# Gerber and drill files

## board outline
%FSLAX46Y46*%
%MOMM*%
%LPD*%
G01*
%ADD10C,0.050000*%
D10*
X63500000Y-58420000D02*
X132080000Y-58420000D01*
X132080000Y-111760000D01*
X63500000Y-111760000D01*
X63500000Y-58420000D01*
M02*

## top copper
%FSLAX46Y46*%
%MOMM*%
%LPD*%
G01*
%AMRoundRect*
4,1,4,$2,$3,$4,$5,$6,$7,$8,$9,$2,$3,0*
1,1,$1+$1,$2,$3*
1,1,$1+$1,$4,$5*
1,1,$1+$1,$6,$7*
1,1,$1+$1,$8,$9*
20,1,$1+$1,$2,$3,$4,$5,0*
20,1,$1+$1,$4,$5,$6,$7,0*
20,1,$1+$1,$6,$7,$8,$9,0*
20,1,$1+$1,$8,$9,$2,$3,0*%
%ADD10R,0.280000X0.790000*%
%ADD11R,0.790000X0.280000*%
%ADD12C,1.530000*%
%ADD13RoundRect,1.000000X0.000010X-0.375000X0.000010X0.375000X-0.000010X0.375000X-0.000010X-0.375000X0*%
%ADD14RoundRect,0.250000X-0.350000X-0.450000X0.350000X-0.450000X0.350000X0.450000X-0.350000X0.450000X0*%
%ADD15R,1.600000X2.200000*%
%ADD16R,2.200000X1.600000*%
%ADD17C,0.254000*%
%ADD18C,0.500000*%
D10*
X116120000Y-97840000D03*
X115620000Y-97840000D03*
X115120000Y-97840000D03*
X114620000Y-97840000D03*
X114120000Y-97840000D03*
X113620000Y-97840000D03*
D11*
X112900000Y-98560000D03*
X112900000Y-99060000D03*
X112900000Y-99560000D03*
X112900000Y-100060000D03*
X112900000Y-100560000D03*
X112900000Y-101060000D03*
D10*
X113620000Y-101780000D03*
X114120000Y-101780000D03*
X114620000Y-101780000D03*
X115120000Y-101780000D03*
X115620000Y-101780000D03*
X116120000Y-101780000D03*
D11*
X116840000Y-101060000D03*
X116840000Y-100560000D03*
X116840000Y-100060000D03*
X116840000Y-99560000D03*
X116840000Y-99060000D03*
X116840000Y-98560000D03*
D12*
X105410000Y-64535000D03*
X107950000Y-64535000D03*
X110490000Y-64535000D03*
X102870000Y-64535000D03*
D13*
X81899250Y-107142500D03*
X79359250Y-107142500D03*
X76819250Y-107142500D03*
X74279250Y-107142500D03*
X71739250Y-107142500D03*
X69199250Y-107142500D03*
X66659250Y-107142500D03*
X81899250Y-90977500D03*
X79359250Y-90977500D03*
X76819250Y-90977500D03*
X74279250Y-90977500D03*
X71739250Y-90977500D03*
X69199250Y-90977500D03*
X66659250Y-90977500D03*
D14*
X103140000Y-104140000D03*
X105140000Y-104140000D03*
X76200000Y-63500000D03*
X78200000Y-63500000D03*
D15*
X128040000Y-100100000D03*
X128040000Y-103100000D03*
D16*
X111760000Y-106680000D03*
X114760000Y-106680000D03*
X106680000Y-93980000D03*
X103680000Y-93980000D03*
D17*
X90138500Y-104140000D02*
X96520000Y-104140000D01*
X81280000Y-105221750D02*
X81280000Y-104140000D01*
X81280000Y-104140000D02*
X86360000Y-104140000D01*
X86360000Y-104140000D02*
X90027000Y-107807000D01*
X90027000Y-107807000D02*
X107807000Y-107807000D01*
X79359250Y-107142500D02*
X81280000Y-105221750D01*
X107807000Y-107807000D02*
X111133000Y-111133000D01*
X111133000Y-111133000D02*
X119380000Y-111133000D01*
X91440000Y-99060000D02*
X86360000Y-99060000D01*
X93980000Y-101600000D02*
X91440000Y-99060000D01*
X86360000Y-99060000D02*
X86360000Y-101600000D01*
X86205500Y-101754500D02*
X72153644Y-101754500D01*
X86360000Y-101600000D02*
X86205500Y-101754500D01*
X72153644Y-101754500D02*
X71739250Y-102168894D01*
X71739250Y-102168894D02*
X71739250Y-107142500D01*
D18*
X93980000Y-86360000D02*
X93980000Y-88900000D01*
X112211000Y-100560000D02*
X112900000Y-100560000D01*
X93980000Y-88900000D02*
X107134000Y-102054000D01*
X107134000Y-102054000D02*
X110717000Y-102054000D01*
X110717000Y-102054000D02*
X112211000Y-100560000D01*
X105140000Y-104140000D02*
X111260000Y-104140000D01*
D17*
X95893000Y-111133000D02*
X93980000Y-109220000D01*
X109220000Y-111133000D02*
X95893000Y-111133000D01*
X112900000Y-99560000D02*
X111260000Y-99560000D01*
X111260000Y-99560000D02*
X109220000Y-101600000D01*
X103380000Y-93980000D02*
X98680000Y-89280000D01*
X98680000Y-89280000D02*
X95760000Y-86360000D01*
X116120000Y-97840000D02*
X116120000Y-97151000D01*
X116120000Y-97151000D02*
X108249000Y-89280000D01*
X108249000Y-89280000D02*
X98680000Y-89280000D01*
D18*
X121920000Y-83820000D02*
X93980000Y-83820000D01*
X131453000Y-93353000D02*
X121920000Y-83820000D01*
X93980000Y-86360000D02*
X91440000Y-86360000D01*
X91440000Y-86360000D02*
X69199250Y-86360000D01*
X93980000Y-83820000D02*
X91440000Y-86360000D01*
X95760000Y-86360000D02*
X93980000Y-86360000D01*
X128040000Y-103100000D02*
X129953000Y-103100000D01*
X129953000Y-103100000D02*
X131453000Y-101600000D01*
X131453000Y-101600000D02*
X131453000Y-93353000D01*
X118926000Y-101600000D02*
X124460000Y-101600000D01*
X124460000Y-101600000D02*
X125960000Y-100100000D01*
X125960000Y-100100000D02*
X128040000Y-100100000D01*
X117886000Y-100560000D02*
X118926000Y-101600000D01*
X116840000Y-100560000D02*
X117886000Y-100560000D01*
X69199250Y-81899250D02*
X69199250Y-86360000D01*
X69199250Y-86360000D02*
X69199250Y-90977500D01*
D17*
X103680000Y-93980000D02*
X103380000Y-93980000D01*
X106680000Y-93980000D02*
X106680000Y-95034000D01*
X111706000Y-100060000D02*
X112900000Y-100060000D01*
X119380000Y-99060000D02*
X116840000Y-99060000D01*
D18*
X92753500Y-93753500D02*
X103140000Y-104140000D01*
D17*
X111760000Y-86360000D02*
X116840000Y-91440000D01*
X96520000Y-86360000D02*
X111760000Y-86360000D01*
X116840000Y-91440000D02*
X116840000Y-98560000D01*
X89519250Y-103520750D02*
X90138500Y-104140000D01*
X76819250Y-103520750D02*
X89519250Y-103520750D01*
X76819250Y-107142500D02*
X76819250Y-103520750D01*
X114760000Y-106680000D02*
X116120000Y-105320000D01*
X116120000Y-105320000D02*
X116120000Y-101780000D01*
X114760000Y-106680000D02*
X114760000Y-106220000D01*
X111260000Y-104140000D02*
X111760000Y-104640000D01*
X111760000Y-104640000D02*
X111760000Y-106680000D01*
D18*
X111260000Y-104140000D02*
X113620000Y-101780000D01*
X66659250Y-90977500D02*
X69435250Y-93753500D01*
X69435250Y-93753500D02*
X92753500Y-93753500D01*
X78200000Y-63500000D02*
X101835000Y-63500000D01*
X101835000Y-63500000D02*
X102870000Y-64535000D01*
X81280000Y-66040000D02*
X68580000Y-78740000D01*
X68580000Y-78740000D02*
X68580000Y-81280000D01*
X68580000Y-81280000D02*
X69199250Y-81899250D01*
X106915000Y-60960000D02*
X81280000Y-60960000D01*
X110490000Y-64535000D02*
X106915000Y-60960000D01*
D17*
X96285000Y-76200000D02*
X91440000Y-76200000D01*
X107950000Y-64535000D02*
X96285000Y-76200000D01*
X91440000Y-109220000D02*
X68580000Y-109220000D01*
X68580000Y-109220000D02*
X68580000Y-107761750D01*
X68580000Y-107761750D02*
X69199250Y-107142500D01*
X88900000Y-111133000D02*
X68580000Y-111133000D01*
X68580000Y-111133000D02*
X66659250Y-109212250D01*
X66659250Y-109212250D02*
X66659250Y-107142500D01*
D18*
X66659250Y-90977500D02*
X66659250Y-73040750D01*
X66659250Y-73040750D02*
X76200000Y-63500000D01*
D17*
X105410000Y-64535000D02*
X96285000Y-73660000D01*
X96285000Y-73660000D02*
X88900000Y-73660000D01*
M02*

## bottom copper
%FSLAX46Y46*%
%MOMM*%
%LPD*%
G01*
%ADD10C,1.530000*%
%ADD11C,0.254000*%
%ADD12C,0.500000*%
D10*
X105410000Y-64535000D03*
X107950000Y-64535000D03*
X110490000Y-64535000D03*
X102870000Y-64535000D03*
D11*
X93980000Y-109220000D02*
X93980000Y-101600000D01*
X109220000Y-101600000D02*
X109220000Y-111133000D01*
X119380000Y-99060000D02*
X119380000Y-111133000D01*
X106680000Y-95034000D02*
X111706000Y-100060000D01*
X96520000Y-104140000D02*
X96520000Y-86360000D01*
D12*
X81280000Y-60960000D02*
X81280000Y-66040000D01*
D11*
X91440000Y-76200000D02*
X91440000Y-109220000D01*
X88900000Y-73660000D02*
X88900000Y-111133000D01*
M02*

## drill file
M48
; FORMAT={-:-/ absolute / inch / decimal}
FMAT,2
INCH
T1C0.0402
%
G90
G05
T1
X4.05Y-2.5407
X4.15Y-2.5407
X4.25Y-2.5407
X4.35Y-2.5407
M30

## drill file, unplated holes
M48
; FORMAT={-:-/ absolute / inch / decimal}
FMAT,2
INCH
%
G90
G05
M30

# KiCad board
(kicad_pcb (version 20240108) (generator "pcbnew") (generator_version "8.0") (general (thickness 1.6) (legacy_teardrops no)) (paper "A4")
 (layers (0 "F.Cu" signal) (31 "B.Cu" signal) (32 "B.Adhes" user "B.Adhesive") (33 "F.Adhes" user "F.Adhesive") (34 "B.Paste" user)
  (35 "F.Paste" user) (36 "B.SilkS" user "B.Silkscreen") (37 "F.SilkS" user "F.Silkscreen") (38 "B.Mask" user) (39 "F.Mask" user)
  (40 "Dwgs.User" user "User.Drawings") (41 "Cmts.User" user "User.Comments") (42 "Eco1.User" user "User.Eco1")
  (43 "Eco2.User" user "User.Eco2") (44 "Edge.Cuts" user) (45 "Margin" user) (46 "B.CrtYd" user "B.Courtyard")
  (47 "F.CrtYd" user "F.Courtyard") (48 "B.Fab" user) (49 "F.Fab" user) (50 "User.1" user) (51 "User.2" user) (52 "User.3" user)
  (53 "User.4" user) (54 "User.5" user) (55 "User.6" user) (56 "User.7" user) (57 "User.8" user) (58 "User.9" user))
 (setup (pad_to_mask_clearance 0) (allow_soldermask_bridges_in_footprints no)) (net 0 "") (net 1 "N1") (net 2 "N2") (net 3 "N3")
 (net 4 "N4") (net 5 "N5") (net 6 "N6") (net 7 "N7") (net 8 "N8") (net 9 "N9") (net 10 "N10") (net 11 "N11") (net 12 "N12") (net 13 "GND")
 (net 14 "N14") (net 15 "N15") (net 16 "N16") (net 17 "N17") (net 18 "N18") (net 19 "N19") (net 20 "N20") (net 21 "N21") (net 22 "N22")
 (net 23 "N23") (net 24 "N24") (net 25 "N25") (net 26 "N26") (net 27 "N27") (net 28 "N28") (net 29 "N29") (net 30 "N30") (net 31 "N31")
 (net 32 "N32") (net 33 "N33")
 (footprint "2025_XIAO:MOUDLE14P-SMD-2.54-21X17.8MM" (layer "F.Cu") (at 84.77925 107.9775 90)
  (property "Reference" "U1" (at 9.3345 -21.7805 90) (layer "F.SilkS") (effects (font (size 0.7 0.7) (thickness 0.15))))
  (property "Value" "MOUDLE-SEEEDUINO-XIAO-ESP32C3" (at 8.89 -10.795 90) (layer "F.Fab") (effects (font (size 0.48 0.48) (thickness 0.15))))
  (pad "1" smd roundrect (at 0.835 -18.12 90) (size 2.75 2) (layers "F.Cu" "F.Paste" "F.Mask") (roundrect_rratio 0.5) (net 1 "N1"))
  (pad "2" smd roundrect (at 0.835 -15.58 90) (size 2.75 2) (layers "F.Cu" "F.Paste" "F.Mask") (roundrect_rratio 0.5) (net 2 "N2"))
  (pad "3" smd roundrect (at 0.835 -13.04 90) (size 2.75 2) (layers "F.Cu" "F.Paste" "F.Mask") (roundrect_rratio 0.5) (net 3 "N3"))
  (pad "4" smd roundrect (at 0.835 -10.5 90) (size 2.75 2) (layers "F.Cu" "F.Paste" "F.Mask") (roundrect_rratio 0.5) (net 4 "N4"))
  (pad "5" smd roundrect (at 0.835 -7.96 90) (size 2.75 2) (layers "F.Cu" "F.Paste" "F.Mask") (roundrect_rratio 0.5) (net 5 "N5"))
  (pad "6" smd roundrect (at 0.835 -5.42 90) (size 2.75 2) (layers "F.Cu" "F.Paste" "F.Mask") (roundrect_rratio 0.5) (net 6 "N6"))
  (pad "7" smd roundrect (at 0.835 -2.88 90) (size 2.75 2) (layers "F.Cu" "F.Paste" "F.Mask") (roundrect_rratio 0.5) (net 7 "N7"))
  (pad "8" smd roundrect (at 17 -2.88 90) (size 2.75 2) (layers "F.Cu" "F.Paste" "F.Mask") (roundrect_rratio 0.5) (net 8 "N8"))
  (pad "9" smd roundrect (at 17 -5.42 90) (size 2.75 2) (layers "F.Cu" "F.Paste" "F.Mask") (roundrect_rratio 0.5) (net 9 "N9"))
  (pad "10" smd roundrect (at 17 -7.96 90) (size 2.75 2) (layers "F.Cu" "F.Paste" "F.Mask") (roundrect_rratio 0.5) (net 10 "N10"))
  (pad "11" smd roundrect (at 17 -10.5 90) (size 2.75 2) (layers "F.Cu" "F.Paste" "F.Mask") (roundrect_rratio 0.5) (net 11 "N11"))
  (pad "12" smd roundrect (at 17 -13.04 90) (size 2.75 2) (layers "F.Cu" "F.Paste" "F.Mask") (roundrect_rratio 0.5) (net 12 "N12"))
  (pad "13" smd roundrect (at 17 -15.58 90) (size 2.75 2) (layers "F.Cu" "F.Paste" "F.Mask") (roundrect_rratio 0.5) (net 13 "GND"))
  (pad "14" smd roundrect (at 17 -18.12 90) (size 2.75 2) (layers "F.Cu" "F.Paste" "F.Mask") (roundrect_rratio 0.5) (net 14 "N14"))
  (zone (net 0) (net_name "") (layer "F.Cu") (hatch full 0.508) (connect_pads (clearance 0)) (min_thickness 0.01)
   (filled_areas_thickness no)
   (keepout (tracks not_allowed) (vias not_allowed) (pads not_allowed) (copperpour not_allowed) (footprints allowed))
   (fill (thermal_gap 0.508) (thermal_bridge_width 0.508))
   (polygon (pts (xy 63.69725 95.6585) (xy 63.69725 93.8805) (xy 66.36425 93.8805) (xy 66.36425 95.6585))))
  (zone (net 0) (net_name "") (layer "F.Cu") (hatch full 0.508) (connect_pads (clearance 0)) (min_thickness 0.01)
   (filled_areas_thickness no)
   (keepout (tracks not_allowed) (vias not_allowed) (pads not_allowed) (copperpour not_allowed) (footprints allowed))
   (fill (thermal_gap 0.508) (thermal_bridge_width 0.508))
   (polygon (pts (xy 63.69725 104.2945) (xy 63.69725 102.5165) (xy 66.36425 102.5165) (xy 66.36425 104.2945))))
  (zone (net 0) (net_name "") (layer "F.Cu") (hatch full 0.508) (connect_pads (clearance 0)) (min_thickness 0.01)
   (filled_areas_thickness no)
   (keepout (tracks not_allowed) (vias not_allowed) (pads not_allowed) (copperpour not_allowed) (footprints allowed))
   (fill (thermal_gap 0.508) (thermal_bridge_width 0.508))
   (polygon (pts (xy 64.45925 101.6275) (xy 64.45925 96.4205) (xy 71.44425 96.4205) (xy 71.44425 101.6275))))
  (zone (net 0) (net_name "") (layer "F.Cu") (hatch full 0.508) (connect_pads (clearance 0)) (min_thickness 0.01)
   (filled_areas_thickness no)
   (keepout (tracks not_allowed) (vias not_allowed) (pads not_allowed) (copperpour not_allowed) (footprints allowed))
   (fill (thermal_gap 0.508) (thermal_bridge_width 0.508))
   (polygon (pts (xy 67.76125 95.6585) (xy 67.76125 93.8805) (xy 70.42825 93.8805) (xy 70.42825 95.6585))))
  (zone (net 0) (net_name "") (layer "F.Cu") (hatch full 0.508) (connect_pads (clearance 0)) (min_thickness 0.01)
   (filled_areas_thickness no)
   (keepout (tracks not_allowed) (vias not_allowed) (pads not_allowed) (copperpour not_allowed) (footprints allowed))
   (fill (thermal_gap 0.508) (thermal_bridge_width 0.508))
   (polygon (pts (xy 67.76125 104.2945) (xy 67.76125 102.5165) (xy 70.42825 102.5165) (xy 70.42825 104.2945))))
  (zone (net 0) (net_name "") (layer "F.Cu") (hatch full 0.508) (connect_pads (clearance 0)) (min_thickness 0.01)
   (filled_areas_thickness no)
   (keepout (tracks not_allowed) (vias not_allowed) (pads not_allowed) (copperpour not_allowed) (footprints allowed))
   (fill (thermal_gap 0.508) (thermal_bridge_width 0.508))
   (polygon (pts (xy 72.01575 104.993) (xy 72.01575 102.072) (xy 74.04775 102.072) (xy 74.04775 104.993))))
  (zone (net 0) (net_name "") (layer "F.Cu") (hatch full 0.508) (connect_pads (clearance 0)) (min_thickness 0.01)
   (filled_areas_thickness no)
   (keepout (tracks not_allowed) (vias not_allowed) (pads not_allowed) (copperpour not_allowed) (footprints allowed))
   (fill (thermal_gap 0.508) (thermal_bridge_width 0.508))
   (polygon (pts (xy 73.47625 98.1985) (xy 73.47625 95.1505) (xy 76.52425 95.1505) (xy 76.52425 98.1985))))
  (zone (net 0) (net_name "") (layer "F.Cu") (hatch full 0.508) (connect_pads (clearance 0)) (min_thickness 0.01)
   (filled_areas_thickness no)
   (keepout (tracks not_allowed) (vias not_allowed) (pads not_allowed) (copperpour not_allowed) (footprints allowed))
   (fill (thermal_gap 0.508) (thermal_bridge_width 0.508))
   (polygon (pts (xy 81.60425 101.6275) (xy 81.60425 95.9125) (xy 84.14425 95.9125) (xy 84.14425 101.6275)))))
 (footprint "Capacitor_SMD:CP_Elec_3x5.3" (layer "F.Cu") (at 113.26 106.68)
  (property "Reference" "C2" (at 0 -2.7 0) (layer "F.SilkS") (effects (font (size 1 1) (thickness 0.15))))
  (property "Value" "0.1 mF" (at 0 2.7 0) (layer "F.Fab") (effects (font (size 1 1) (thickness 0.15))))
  (pad "1" smd rect (at -1.5 0) (size 2.2 1.6) (layers "F.Cu" "F.Paste" "F.Mask") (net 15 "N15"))
  (pad "2" smd rect (at 1.5 0) (size 2.2 1.6) (layers "F.Cu" "F.Paste" "F.Mask") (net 13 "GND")))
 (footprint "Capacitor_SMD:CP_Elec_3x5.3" (layer "F.Cu") (at 128.04 101.6 -90)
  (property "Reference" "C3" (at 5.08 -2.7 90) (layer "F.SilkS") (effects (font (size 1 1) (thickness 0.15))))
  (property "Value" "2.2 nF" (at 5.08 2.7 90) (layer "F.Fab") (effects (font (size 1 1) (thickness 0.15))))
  (pad "1" smd rect (at -1.5 0 270) (size 2.2 1.6) (layers "F.Cu" "F.Paste" "F.Mask") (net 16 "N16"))
  (pad "2" smd rect (at 1.5 0 270) (size 2.2 1.6) (layers "F.Cu" "F.Paste" "F.Mask") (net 13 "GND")))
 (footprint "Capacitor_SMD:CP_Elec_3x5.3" (layer "F.Cu") (at 105.18 93.98 180)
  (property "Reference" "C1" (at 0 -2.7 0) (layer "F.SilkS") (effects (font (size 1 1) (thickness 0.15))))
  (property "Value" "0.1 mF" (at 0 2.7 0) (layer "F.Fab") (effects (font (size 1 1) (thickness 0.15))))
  (pad "1" smd rect (at -1.5 0 180) (size 2.2 1.6) (layers "F.Cu" "F.Paste" "F.Mask") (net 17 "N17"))
  (pad "2" smd rect (at 1.5 0 180) (size 2.2 1.6) (layers "F.Cu" "F.Paste" "F.Mask") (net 13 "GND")))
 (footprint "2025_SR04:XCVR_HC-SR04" (layer "F.Cu") (at 106.68 64.535)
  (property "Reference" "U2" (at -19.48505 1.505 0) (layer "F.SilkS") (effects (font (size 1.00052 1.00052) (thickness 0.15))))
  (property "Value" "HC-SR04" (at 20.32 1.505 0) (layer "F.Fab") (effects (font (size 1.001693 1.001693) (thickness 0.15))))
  (pad "1" thru_hole circle (at -3.81 0) (size 1.53 1.53) (drill 1.02) (layers "*.Cu" "*.Mask") (remove_unused_layers no) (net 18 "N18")
   (solder_mask_margin 0.102))
  (pad "2" thru_hole circle (at -1.27 0) (size 1.53 1.53) (drill 1.02) (layers "*.Cu" "*.Mask") (remove_unused_layers no) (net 1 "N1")
   (solder_mask_margin 0.102))
  (pad "3" thru_hole circle (at 1.27 0) (size 1.53 1.53) (drill 1.02) (layers "*.Cu" "*.Mask") (remove_unused_layers no) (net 2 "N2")
   (solder_mask_margin 0.102))
  (pad "4" thru_hole circle (at 3.81 0) (size 1.53 1.53) (drill 1.02) (layers "*.Cu" "*.Mask") (remove_unused_layers no) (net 13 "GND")
   (solder_mask_margin 0.102)))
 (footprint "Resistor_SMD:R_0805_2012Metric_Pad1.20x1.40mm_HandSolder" (layer "F.Cu") (at 77.2 63.5)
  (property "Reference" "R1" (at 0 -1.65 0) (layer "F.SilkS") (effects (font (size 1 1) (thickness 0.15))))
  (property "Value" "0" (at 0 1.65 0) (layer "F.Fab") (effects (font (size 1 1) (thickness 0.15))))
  (pad "1" smd roundrect (at -1 0) (size 1.2 1.4) (layers "F.Cu" "F.Paste" "F.Mask") (roundrect_rratio 0.208333) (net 14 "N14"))
  (pad "2" smd roundrect (at 1 0) (size 1.2 1.4) (layers "F.Cu" "F.Paste" "F.Mask") (roundrect_rratio 0.208333) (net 18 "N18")))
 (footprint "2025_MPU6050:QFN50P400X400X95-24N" (layer "F.Cu") (at 114.87 99.81 -90)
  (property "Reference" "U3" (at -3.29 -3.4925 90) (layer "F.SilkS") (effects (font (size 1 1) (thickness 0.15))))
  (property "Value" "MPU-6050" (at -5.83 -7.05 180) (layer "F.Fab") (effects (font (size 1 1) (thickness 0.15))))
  (pad "1" smd rect (at -1.97 -1.25 270) (size 0.79 0.28) (layers "F.Cu" "F.Paste" "F.Mask") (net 13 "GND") (solder_mask_margin 0.102))
  (pad "2" smd rect (at -1.97 -0.75 270) (size 0.79 0.28) (layers "F.Cu" "F.Paste" "F.Mask") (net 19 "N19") (solder_mask_margin 0.102))
  (pad "3" smd rect (at -1.97 -0.25 270) (size 0.79 0.28) (layers "F.Cu" "F.Paste" "F.Mask") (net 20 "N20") (solder_mask_margin 0.102))
  (pad "4" smd rect (at -1.97 0.25 270) (size 0.79 0.28) (layers "F.Cu" "F.Paste" "F.Mask") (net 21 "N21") (solder_mask_margin 0.102))
  (pad "5" smd rect (at -1.97 0.75 270) (size 0.79 0.28) (layers "F.Cu" "F.Paste" "F.Mask") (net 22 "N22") (solder_mask_margin 0.102))
  (pad "6" smd rect (at -1.97 1.25 270) (size 0.79 0.28) (layers "F.Cu" "F.Paste" "F.Mask") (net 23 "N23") (solder_mask_margin 0.102))
  (pad "7" smd rect (at -1.25 1.97 270) (size 0.28 0.79) (layers "F.Cu" "F.Paste" "F.Mask") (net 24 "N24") (solder_mask_margin 0.102))
  (pad "8" smd rect (at -0.75 1.97 270) (size 0.28 0.79) (layers "F.Cu" "F.Paste" "F.Mask") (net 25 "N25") (solder_mask_margin 0.102))
  (pad "9" smd rect (at -0.25 1.97 270) (size 0.28 0.79) (layers "F.Cu" "F.Paste" "F.Mask") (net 3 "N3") (solder_mask_margin 0.102))
  (pad "10" smd rect (at 0.25 1.97 270) (size 0.28 0.79) (layers "F.Cu" "F.Paste" "F.Mask") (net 17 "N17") (solder_mask_margin 0.102))
  (pad "11" smd rect (at 0.75 1.97 270) (size 0.28 0.79) (layers "F.Cu" "F.Paste" "F.Mask") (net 13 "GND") (solder_mask_margin 0.102))
  (pad "12" smd rect (at 1.25 1.97 270) (size 0.28 0.79) (layers "F.Cu" "F.Paste" "F.Mask") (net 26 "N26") (solder_mask_margin 0.102))
  (pad "13" smd rect (at 1.97 1.25 270) (size 0.79 0.28) (layers "F.Cu" "F.Paste" "F.Mask") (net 15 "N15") (solder_mask_margin 0.102))
  (pad "14" smd rect (at 1.97 0.75 270) (size 0.79 0.28) (layers "F.Cu" "F.Paste" "F.Mask") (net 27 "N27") (solder_mask_margin 0.102))
  (pad "15" smd rect (at 1.97 0.25 270) (size 0.79 0.28) (layers "F.Cu" "F.Paste" "F.Mask") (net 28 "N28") (solder_mask_margin 0.102))
  (pad "16" smd rect (at 1.97 -0.25 270) (size 0.79 0.28) (layers "F.Cu" "F.Paste" "F.Mask") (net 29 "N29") (solder_mask_margin 0.102))
  (pad "17" smd rect (at 1.97 -0.75 270) (size 0.79 0.28) (layers "F.Cu" "F.Paste" "F.Mask") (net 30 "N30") (solder_mask_margin 0.102))
  (pad "18" smd rect (at 1.97 -1.25 270) (size 0.79 0.28) (layers "F.Cu" "F.Paste" "F.Mask") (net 13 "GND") (solder_mask_margin 0.102))
  (pad "19" smd rect (at 1.25 -1.97 270) (size 0.28 0.79) (layers "F.Cu" "F.Paste" "F.Mask") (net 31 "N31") (solder_mask_margin 0.102))
  (pad "20" smd rect (at 0.75 -1.97 270) (size 0.28 0.79) (layers "F.Cu" "F.Paste" "F.Mask") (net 16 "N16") (solder_mask_margin 0.102))
  (pad "21" smd rect (at 0.25 -1.97 270) (size 0.28 0.79) (layers "F.Cu" "F.Paste" "F.Mask") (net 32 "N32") (solder_mask_margin 0.102))
  (pad "22" smd rect (at -0.25 -1.97 270) (size 0.28 0.79) (layers "F.Cu" "F.Paste" "F.Mask") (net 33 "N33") (solder_mask_margin 0.102))
  (pad "23" smd rect (at -0.75 -1.97 270) (size 0.28 0.79) (layers "F.Cu" "F.Paste" "F.Mask") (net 6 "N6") (solder_mask_margin 0.102))
  (pad "24" smd rect (at -1.25 -1.97 270) (size 0.28 0.79) (layers "F.Cu" "F.Paste" "F.Mask") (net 5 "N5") (solder_mask_margin 0.102))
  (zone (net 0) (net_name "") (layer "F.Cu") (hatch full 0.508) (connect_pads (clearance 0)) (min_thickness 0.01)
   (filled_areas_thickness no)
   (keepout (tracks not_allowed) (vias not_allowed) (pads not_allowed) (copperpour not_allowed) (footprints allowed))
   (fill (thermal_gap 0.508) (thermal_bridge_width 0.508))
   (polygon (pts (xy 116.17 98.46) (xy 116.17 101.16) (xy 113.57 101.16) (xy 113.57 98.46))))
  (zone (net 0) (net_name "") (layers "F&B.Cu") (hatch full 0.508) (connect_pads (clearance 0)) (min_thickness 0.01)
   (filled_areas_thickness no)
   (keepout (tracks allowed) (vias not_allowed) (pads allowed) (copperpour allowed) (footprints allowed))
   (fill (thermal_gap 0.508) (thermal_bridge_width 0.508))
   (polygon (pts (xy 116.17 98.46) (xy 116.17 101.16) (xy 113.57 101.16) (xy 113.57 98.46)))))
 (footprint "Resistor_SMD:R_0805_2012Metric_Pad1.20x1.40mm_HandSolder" (layer "F.Cu") (at 104.14 104.14)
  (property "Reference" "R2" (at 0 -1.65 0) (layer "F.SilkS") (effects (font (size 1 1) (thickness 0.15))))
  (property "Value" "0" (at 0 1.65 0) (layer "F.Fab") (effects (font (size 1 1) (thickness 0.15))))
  (pad "1" smd roundrect (at -1 0) (size 1.2 1.4) (layers "F.Cu" "F.Paste" "F.Mask") (roundrect_rratio 0.208333) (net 14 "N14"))
  (pad "2" smd roundrect (at 1 0) (size 1.2 1.4) (layers "F.Cu" "F.Paste" "F.Mask") (roundrect_rratio 0.208333) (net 15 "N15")))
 (gr_rect (start 63.5 58.42) (end 132.08 111.76) (stroke (width 0.05) (type default)) (fill none) (layer "Edge.Cuts"))
 (segment (start 105.41 64.535) (end 96.285 73.66) (width 0.254) (layer "F.Cu") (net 1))
 (segment (start 88.9 111.133) (end 68.58 111.133) (width 0.254) (layer "F.Cu") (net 1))
 (segment (start 66.65925 109.21225) (end 66.65925 107.1425) (width 0.254) (layer "F.Cu") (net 1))
 (segment (start 68.58 111.133) (end 66.65925 109.21225) (width 0.254) (layer "F.Cu") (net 1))
 (segment (start 96.285 73.66) (end 88.9 73.66) (width 0.254) (layer "F.Cu") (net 1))
 (segment (start 88.9 73.66) (end 88.9 111.133) (width 0.254) (layer "B.Cu") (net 1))
 (segment (start 96.285 76.2) (end 91.44 76.2) (width 0.254) (layer "F.Cu") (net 2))
 (segment (start 91.44 109.22) (end 68.58 109.22) (width 0.254) (layer "F.Cu") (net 2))
 (segment (start 68.58 107.76175) (end 69.19925 107.1425) (width 0.254) (layer "F.Cu") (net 2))
 (segment (start 68.58 109.22) (end 68.58 107.76175) (width 0.254) (layer "F.Cu") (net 2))
 (segment (start 107.95 64.535) (end 96.285 76.2) (width 0.254) (layer "F.Cu") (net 2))
 (segment (start 91.44 76.2) (end 91.44 109.22) (width 0.254) (layer "B.Cu") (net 2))
 (segment (start 101.835 63.5) (end 102.87 64.535) (width 0.5) (layer "F.Cu") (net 18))
 (segment (start 78.2 63.5) (end 101.835 63.5) (width 0.5) (layer "F.Cu") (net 18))
 (segment (start 68.58 81.28) (end 69.19925 81.89925) (width 0.5) (layer "F.Cu") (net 13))
 (segment (start 112.211 100.56) (end 112.9 100.56) (width 0.5) (layer "F.Cu") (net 13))
 (segment (start 81.28 66.04) (end 68.58 78.74) (width 0.5) (layer "F.Cu") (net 13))
 (segment (start 106.915 60.96) (end 81.28 60.96) (width 0.5) (layer "F.Cu") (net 13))
 (segment (start 69.19925 86.36) (end 69.19925 90.9775) (width 0.5) (layer "F.Cu") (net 13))
 (segment (start 93.98 88.9) (end 107.134 102.054) (width 0.5) (layer "F.Cu") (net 13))
 (segment (start 93.98 86.36) (end 93.98 88.9) (width 0.5) (layer "F.Cu") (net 13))
 (segment (start 131.453 101.6) (end 131.453 93.353) (width 0.5) (layer "F.Cu") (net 13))
 (segment (start 116.12 97.151) (end 108.249 89.28) (width 0.254) (layer "F.Cu") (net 13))
 (segment (start 116.12 105.32) (end 116.12 101.78) (width 0.254) (layer "F.Cu") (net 13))
 (segment (start 116.12 97.84) (end 116.12 97.151) (width 0.254) (layer "F.Cu") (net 13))
 (segment (start 108.249 89.28) (end 98.68 89.28) (width 0.254) (layer "F.Cu") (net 13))
 (segment (start 121.92 83.82) (end 93.98 83.82) (width 0.5) (layer "F.Cu") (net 13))
 (segment (start 93.98 86.36) (end 91.44 86.36) (width 0.5) (layer "F.Cu") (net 13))
 (segment (start 98.68 89.28) (end 95.76 86.36) (width 0.254) (layer "F.Cu") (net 13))
 (segment (start 128.04 103.1) (end 129.953 103.1) (width 0.5) (layer "F.Cu") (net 13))
 (segment (start 129.953 103.1) (end 131.453 101.6) (width 0.5) (layer "F.Cu") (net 13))
 (segment (start 95.76 86.36) (end 93.98 86.36) (width 0.5) (layer "F.Cu") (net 13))
 (segment (start 110.717 102.054) (end 112.211 100.56) (width 0.5) (layer "F.Cu") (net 13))
 (segment (start 91.44 86.36) (end 69.19925 86.36) (width 0.5) (layer "F.Cu") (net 13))
 (segment (start 103.68 93.98) (end 103.38 93.98) (width 0.254) (layer "F.Cu") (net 13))
 (segment (start 69.19925 81.89925) (end 69.19925 86.36) (width 0.5) (layer "F.Cu") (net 13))
 (segment (start 110.49 64.535) (end 106.915 60.96) (width 0.5) (layer "F.Cu") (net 13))
 (segment (start 107.134 102.054) (end 110.717 102.054) (width 0.5) (layer "F.Cu") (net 13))
 (segment (start 131.453 93.353) (end 121.92 83.82) (width 0.5) (layer "F.Cu") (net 13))
 (segment (start 114.76 106.68) (end 114.76 106.22) (width 0.254) (layer "F.Cu") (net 13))
 (segment (start 93.98 83.82) (end 91.44 86.36) (width 0.5) (layer "F.Cu") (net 13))
 (segment (start 68.58 78.74) (end 68.58 81.28) (width 0.5) (layer "F.Cu") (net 13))
 (segment (start 103.38 93.98) (end 98.68 89.28) (width 0.254) (layer "F.Cu") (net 13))
 (segment (start 114.76 106.68) (end 116.12 105.32) (width 0.254) (layer "F.Cu") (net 13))
 (segment (start 81.28 60.96) (end 81.28 66.04) (width 0.5) (layer "B.Cu") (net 13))
 (segment (start 106.68 93.98) (end 106.68 95.034) (width 0.254) (layer "F.Cu") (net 17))
 (segment (start 111.706 100.06) (end 112.9 100.06) (width 0.254) (layer "F.Cu") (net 17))
 (segment (start 106.68 95.034) (end 111.706 100.06) (width 0.254) (layer "B.Cu") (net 17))
 (segment (start 125.96 100.1) (end 128.04 100.1) (width 0.5) (layer "F.Cu") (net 16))
 (segment (start 124.46 101.6) (end 125.96 100.1) (width 0.5) (layer "F.Cu") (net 16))
 (segment (start 116.84 100.56) (end 117.886 100.56) (width 0.5) (layer "F.Cu") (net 16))
 (segment (start 118.926 101.6) (end 124.46 101.6) (width 0.5) (layer "F.Cu") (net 16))
 (segment (start 117.886 100.56) (end 118.926 101.6) (width 0.5) (layer "F.Cu") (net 16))
 (segment (start 86.36 104.14) (end 90.027 107.807) (width 0.254) (layer "F.Cu") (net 6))
 (segment (start 81.28 104.14) (end 86.36 104.14) (width 0.254) (layer "F.Cu") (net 6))
 (segment (start 79.35925 107.1425) (end 81.28 105.22175) (width 0.254) (layer "F.Cu") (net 6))
 (segment (start 81.28 105.22175) (end 81.28 104.14) (width 0.254) (layer "F.Cu") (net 6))
 (segment (start 90.027 107.807) (end 107.807 107.807) (width 0.254) (layer "F.Cu") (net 6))
 (segment (start 111.133 111.133) (end 119.38 111.133) (width 0.254) (layer "F.Cu") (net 6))
 (segment (start 119.38 99.06) (end 116.84 99.06) (width 0.254) (layer "F.Cu") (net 6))
 (segment (start 107.807 107.807) (end 111.133 111.133) (width 0.254) (layer "F.Cu") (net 6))
 (segment (start 119.38 99.06) (end 119.38 111.133) (width 0.254) (layer "B.Cu") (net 6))
 (segment (start 95.893 111.133) (end 93.98 109.22) (width 0.254) (layer "F.Cu") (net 3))
 (segment (start 111.26 99.56) (end 109.22 101.6) (width 0.254) (layer "F.Cu") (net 3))
 (segment (start 91.44 99.06) (end 86.36 99.06) (width 0.254) (layer "F.Cu") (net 3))
 (segment (start 71.73925 102.168894) (end 71.73925 107.1425) (width 0.254) (layer "F.Cu") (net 3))
 (segment (start 86.36 101.6) (end 86.2055 101.7545) (width 0.254) (layer "F.Cu") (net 3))
 (segment (start 109.22 111.133) (end 95.893 111.133) (width 0.254) (layer "F.Cu") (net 3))
 (segment (start 86.2055 101.7545) (end 72.153644 101.7545) (width 0.254) (layer "F.Cu") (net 3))
 (segment (start 86.36 99.06) (end 86.36 101.6) (width 0.254) (layer "F.Cu") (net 3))
 (segment (start 72.153644 101.7545) (end 71.73925 102.168894) (width 0.254) (layer "F.Cu") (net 3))
 (segment (start 112.9 99.56) (end 111.26 99.56) (width 0.254) (layer "F.Cu") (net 3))
 (segment (start 93.98 101.6) (end 91.44 99.06) (width 0.254) (layer "F.Cu") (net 3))
 (segment (start 93.98 109.22) (end 93.98 101.6) (width 0.254) (layer "B.Cu") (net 3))
 (segment (start 109.22 101.6) (end 109.22 111.133) (width 0.254) (layer "B.Cu") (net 3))
 (segment (start 111.26 104.14) (end 111.76 104.64) (width 0.254) (layer "F.Cu") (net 15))
 (segment (start 105.14 104.14) (end 111.26 104.14) (width 0.5) (layer "F.Cu") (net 15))
 (segment (start 111.76 104.64) (end 111.76 106.68) (width 0.254) (layer "F.Cu") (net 15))
 (segment (start 111.26 104.14) (end 113.62 101.78) (width 0.5) (layer "F.Cu") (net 15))
 (segment (start 96.52 86.36) (end 111.76 86.36) (width 0.254) (layer "F.Cu") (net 5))
 (segment (start 116.84 91.44) (end 116.84 98.56) (width 0.254) (layer "F.Cu") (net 5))
 (segment (start 90.1385 104.14) (end 96.52 104.14) (width 0.254) (layer "F.Cu") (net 5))
 (segment (start 76.81925 103.52075) (end 89.51925 103.52075) (width 0.254) (layer "F.Cu") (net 5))
 (segment (start 76.81925 107.1425) (end 76.81925 103.52075) (width 0.254) (layer "F.Cu") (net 5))
 (segment (start 89.51925 103.52075) (end 90.1385 104.14) (width 0.254) (layer "F.Cu") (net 5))
 (segment (start 111.76 86.36) (end 116.84 91.44) (width 0.254) (layer "F.Cu") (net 5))
 (segment (start 96.52 104.14) (end 96.52 86.36) (width 0.254) (layer "B.Cu") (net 5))
 (segment (start 66.65925 90.9775) (end 69.43525 93.7535) (width 0.5) (layer "F.Cu") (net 14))
 (segment (start 66.65925 90.9775) (end 66.65925 73.04075) (width 0.5) (layer "F.Cu") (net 14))
 (segment (start 69.43525 93.7535) (end 92.7535 93.7535) (width 0.5) (layer "F.Cu") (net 14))
 (segment (start 92.7535 93.7535) (end 103.14 104.14) (width 0.5) (layer "F.Cu") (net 14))
 (segment (start 66.65925 73.04075) (end 76.2 63.5) (width 0.5) (layer "F.Cu") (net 14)))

